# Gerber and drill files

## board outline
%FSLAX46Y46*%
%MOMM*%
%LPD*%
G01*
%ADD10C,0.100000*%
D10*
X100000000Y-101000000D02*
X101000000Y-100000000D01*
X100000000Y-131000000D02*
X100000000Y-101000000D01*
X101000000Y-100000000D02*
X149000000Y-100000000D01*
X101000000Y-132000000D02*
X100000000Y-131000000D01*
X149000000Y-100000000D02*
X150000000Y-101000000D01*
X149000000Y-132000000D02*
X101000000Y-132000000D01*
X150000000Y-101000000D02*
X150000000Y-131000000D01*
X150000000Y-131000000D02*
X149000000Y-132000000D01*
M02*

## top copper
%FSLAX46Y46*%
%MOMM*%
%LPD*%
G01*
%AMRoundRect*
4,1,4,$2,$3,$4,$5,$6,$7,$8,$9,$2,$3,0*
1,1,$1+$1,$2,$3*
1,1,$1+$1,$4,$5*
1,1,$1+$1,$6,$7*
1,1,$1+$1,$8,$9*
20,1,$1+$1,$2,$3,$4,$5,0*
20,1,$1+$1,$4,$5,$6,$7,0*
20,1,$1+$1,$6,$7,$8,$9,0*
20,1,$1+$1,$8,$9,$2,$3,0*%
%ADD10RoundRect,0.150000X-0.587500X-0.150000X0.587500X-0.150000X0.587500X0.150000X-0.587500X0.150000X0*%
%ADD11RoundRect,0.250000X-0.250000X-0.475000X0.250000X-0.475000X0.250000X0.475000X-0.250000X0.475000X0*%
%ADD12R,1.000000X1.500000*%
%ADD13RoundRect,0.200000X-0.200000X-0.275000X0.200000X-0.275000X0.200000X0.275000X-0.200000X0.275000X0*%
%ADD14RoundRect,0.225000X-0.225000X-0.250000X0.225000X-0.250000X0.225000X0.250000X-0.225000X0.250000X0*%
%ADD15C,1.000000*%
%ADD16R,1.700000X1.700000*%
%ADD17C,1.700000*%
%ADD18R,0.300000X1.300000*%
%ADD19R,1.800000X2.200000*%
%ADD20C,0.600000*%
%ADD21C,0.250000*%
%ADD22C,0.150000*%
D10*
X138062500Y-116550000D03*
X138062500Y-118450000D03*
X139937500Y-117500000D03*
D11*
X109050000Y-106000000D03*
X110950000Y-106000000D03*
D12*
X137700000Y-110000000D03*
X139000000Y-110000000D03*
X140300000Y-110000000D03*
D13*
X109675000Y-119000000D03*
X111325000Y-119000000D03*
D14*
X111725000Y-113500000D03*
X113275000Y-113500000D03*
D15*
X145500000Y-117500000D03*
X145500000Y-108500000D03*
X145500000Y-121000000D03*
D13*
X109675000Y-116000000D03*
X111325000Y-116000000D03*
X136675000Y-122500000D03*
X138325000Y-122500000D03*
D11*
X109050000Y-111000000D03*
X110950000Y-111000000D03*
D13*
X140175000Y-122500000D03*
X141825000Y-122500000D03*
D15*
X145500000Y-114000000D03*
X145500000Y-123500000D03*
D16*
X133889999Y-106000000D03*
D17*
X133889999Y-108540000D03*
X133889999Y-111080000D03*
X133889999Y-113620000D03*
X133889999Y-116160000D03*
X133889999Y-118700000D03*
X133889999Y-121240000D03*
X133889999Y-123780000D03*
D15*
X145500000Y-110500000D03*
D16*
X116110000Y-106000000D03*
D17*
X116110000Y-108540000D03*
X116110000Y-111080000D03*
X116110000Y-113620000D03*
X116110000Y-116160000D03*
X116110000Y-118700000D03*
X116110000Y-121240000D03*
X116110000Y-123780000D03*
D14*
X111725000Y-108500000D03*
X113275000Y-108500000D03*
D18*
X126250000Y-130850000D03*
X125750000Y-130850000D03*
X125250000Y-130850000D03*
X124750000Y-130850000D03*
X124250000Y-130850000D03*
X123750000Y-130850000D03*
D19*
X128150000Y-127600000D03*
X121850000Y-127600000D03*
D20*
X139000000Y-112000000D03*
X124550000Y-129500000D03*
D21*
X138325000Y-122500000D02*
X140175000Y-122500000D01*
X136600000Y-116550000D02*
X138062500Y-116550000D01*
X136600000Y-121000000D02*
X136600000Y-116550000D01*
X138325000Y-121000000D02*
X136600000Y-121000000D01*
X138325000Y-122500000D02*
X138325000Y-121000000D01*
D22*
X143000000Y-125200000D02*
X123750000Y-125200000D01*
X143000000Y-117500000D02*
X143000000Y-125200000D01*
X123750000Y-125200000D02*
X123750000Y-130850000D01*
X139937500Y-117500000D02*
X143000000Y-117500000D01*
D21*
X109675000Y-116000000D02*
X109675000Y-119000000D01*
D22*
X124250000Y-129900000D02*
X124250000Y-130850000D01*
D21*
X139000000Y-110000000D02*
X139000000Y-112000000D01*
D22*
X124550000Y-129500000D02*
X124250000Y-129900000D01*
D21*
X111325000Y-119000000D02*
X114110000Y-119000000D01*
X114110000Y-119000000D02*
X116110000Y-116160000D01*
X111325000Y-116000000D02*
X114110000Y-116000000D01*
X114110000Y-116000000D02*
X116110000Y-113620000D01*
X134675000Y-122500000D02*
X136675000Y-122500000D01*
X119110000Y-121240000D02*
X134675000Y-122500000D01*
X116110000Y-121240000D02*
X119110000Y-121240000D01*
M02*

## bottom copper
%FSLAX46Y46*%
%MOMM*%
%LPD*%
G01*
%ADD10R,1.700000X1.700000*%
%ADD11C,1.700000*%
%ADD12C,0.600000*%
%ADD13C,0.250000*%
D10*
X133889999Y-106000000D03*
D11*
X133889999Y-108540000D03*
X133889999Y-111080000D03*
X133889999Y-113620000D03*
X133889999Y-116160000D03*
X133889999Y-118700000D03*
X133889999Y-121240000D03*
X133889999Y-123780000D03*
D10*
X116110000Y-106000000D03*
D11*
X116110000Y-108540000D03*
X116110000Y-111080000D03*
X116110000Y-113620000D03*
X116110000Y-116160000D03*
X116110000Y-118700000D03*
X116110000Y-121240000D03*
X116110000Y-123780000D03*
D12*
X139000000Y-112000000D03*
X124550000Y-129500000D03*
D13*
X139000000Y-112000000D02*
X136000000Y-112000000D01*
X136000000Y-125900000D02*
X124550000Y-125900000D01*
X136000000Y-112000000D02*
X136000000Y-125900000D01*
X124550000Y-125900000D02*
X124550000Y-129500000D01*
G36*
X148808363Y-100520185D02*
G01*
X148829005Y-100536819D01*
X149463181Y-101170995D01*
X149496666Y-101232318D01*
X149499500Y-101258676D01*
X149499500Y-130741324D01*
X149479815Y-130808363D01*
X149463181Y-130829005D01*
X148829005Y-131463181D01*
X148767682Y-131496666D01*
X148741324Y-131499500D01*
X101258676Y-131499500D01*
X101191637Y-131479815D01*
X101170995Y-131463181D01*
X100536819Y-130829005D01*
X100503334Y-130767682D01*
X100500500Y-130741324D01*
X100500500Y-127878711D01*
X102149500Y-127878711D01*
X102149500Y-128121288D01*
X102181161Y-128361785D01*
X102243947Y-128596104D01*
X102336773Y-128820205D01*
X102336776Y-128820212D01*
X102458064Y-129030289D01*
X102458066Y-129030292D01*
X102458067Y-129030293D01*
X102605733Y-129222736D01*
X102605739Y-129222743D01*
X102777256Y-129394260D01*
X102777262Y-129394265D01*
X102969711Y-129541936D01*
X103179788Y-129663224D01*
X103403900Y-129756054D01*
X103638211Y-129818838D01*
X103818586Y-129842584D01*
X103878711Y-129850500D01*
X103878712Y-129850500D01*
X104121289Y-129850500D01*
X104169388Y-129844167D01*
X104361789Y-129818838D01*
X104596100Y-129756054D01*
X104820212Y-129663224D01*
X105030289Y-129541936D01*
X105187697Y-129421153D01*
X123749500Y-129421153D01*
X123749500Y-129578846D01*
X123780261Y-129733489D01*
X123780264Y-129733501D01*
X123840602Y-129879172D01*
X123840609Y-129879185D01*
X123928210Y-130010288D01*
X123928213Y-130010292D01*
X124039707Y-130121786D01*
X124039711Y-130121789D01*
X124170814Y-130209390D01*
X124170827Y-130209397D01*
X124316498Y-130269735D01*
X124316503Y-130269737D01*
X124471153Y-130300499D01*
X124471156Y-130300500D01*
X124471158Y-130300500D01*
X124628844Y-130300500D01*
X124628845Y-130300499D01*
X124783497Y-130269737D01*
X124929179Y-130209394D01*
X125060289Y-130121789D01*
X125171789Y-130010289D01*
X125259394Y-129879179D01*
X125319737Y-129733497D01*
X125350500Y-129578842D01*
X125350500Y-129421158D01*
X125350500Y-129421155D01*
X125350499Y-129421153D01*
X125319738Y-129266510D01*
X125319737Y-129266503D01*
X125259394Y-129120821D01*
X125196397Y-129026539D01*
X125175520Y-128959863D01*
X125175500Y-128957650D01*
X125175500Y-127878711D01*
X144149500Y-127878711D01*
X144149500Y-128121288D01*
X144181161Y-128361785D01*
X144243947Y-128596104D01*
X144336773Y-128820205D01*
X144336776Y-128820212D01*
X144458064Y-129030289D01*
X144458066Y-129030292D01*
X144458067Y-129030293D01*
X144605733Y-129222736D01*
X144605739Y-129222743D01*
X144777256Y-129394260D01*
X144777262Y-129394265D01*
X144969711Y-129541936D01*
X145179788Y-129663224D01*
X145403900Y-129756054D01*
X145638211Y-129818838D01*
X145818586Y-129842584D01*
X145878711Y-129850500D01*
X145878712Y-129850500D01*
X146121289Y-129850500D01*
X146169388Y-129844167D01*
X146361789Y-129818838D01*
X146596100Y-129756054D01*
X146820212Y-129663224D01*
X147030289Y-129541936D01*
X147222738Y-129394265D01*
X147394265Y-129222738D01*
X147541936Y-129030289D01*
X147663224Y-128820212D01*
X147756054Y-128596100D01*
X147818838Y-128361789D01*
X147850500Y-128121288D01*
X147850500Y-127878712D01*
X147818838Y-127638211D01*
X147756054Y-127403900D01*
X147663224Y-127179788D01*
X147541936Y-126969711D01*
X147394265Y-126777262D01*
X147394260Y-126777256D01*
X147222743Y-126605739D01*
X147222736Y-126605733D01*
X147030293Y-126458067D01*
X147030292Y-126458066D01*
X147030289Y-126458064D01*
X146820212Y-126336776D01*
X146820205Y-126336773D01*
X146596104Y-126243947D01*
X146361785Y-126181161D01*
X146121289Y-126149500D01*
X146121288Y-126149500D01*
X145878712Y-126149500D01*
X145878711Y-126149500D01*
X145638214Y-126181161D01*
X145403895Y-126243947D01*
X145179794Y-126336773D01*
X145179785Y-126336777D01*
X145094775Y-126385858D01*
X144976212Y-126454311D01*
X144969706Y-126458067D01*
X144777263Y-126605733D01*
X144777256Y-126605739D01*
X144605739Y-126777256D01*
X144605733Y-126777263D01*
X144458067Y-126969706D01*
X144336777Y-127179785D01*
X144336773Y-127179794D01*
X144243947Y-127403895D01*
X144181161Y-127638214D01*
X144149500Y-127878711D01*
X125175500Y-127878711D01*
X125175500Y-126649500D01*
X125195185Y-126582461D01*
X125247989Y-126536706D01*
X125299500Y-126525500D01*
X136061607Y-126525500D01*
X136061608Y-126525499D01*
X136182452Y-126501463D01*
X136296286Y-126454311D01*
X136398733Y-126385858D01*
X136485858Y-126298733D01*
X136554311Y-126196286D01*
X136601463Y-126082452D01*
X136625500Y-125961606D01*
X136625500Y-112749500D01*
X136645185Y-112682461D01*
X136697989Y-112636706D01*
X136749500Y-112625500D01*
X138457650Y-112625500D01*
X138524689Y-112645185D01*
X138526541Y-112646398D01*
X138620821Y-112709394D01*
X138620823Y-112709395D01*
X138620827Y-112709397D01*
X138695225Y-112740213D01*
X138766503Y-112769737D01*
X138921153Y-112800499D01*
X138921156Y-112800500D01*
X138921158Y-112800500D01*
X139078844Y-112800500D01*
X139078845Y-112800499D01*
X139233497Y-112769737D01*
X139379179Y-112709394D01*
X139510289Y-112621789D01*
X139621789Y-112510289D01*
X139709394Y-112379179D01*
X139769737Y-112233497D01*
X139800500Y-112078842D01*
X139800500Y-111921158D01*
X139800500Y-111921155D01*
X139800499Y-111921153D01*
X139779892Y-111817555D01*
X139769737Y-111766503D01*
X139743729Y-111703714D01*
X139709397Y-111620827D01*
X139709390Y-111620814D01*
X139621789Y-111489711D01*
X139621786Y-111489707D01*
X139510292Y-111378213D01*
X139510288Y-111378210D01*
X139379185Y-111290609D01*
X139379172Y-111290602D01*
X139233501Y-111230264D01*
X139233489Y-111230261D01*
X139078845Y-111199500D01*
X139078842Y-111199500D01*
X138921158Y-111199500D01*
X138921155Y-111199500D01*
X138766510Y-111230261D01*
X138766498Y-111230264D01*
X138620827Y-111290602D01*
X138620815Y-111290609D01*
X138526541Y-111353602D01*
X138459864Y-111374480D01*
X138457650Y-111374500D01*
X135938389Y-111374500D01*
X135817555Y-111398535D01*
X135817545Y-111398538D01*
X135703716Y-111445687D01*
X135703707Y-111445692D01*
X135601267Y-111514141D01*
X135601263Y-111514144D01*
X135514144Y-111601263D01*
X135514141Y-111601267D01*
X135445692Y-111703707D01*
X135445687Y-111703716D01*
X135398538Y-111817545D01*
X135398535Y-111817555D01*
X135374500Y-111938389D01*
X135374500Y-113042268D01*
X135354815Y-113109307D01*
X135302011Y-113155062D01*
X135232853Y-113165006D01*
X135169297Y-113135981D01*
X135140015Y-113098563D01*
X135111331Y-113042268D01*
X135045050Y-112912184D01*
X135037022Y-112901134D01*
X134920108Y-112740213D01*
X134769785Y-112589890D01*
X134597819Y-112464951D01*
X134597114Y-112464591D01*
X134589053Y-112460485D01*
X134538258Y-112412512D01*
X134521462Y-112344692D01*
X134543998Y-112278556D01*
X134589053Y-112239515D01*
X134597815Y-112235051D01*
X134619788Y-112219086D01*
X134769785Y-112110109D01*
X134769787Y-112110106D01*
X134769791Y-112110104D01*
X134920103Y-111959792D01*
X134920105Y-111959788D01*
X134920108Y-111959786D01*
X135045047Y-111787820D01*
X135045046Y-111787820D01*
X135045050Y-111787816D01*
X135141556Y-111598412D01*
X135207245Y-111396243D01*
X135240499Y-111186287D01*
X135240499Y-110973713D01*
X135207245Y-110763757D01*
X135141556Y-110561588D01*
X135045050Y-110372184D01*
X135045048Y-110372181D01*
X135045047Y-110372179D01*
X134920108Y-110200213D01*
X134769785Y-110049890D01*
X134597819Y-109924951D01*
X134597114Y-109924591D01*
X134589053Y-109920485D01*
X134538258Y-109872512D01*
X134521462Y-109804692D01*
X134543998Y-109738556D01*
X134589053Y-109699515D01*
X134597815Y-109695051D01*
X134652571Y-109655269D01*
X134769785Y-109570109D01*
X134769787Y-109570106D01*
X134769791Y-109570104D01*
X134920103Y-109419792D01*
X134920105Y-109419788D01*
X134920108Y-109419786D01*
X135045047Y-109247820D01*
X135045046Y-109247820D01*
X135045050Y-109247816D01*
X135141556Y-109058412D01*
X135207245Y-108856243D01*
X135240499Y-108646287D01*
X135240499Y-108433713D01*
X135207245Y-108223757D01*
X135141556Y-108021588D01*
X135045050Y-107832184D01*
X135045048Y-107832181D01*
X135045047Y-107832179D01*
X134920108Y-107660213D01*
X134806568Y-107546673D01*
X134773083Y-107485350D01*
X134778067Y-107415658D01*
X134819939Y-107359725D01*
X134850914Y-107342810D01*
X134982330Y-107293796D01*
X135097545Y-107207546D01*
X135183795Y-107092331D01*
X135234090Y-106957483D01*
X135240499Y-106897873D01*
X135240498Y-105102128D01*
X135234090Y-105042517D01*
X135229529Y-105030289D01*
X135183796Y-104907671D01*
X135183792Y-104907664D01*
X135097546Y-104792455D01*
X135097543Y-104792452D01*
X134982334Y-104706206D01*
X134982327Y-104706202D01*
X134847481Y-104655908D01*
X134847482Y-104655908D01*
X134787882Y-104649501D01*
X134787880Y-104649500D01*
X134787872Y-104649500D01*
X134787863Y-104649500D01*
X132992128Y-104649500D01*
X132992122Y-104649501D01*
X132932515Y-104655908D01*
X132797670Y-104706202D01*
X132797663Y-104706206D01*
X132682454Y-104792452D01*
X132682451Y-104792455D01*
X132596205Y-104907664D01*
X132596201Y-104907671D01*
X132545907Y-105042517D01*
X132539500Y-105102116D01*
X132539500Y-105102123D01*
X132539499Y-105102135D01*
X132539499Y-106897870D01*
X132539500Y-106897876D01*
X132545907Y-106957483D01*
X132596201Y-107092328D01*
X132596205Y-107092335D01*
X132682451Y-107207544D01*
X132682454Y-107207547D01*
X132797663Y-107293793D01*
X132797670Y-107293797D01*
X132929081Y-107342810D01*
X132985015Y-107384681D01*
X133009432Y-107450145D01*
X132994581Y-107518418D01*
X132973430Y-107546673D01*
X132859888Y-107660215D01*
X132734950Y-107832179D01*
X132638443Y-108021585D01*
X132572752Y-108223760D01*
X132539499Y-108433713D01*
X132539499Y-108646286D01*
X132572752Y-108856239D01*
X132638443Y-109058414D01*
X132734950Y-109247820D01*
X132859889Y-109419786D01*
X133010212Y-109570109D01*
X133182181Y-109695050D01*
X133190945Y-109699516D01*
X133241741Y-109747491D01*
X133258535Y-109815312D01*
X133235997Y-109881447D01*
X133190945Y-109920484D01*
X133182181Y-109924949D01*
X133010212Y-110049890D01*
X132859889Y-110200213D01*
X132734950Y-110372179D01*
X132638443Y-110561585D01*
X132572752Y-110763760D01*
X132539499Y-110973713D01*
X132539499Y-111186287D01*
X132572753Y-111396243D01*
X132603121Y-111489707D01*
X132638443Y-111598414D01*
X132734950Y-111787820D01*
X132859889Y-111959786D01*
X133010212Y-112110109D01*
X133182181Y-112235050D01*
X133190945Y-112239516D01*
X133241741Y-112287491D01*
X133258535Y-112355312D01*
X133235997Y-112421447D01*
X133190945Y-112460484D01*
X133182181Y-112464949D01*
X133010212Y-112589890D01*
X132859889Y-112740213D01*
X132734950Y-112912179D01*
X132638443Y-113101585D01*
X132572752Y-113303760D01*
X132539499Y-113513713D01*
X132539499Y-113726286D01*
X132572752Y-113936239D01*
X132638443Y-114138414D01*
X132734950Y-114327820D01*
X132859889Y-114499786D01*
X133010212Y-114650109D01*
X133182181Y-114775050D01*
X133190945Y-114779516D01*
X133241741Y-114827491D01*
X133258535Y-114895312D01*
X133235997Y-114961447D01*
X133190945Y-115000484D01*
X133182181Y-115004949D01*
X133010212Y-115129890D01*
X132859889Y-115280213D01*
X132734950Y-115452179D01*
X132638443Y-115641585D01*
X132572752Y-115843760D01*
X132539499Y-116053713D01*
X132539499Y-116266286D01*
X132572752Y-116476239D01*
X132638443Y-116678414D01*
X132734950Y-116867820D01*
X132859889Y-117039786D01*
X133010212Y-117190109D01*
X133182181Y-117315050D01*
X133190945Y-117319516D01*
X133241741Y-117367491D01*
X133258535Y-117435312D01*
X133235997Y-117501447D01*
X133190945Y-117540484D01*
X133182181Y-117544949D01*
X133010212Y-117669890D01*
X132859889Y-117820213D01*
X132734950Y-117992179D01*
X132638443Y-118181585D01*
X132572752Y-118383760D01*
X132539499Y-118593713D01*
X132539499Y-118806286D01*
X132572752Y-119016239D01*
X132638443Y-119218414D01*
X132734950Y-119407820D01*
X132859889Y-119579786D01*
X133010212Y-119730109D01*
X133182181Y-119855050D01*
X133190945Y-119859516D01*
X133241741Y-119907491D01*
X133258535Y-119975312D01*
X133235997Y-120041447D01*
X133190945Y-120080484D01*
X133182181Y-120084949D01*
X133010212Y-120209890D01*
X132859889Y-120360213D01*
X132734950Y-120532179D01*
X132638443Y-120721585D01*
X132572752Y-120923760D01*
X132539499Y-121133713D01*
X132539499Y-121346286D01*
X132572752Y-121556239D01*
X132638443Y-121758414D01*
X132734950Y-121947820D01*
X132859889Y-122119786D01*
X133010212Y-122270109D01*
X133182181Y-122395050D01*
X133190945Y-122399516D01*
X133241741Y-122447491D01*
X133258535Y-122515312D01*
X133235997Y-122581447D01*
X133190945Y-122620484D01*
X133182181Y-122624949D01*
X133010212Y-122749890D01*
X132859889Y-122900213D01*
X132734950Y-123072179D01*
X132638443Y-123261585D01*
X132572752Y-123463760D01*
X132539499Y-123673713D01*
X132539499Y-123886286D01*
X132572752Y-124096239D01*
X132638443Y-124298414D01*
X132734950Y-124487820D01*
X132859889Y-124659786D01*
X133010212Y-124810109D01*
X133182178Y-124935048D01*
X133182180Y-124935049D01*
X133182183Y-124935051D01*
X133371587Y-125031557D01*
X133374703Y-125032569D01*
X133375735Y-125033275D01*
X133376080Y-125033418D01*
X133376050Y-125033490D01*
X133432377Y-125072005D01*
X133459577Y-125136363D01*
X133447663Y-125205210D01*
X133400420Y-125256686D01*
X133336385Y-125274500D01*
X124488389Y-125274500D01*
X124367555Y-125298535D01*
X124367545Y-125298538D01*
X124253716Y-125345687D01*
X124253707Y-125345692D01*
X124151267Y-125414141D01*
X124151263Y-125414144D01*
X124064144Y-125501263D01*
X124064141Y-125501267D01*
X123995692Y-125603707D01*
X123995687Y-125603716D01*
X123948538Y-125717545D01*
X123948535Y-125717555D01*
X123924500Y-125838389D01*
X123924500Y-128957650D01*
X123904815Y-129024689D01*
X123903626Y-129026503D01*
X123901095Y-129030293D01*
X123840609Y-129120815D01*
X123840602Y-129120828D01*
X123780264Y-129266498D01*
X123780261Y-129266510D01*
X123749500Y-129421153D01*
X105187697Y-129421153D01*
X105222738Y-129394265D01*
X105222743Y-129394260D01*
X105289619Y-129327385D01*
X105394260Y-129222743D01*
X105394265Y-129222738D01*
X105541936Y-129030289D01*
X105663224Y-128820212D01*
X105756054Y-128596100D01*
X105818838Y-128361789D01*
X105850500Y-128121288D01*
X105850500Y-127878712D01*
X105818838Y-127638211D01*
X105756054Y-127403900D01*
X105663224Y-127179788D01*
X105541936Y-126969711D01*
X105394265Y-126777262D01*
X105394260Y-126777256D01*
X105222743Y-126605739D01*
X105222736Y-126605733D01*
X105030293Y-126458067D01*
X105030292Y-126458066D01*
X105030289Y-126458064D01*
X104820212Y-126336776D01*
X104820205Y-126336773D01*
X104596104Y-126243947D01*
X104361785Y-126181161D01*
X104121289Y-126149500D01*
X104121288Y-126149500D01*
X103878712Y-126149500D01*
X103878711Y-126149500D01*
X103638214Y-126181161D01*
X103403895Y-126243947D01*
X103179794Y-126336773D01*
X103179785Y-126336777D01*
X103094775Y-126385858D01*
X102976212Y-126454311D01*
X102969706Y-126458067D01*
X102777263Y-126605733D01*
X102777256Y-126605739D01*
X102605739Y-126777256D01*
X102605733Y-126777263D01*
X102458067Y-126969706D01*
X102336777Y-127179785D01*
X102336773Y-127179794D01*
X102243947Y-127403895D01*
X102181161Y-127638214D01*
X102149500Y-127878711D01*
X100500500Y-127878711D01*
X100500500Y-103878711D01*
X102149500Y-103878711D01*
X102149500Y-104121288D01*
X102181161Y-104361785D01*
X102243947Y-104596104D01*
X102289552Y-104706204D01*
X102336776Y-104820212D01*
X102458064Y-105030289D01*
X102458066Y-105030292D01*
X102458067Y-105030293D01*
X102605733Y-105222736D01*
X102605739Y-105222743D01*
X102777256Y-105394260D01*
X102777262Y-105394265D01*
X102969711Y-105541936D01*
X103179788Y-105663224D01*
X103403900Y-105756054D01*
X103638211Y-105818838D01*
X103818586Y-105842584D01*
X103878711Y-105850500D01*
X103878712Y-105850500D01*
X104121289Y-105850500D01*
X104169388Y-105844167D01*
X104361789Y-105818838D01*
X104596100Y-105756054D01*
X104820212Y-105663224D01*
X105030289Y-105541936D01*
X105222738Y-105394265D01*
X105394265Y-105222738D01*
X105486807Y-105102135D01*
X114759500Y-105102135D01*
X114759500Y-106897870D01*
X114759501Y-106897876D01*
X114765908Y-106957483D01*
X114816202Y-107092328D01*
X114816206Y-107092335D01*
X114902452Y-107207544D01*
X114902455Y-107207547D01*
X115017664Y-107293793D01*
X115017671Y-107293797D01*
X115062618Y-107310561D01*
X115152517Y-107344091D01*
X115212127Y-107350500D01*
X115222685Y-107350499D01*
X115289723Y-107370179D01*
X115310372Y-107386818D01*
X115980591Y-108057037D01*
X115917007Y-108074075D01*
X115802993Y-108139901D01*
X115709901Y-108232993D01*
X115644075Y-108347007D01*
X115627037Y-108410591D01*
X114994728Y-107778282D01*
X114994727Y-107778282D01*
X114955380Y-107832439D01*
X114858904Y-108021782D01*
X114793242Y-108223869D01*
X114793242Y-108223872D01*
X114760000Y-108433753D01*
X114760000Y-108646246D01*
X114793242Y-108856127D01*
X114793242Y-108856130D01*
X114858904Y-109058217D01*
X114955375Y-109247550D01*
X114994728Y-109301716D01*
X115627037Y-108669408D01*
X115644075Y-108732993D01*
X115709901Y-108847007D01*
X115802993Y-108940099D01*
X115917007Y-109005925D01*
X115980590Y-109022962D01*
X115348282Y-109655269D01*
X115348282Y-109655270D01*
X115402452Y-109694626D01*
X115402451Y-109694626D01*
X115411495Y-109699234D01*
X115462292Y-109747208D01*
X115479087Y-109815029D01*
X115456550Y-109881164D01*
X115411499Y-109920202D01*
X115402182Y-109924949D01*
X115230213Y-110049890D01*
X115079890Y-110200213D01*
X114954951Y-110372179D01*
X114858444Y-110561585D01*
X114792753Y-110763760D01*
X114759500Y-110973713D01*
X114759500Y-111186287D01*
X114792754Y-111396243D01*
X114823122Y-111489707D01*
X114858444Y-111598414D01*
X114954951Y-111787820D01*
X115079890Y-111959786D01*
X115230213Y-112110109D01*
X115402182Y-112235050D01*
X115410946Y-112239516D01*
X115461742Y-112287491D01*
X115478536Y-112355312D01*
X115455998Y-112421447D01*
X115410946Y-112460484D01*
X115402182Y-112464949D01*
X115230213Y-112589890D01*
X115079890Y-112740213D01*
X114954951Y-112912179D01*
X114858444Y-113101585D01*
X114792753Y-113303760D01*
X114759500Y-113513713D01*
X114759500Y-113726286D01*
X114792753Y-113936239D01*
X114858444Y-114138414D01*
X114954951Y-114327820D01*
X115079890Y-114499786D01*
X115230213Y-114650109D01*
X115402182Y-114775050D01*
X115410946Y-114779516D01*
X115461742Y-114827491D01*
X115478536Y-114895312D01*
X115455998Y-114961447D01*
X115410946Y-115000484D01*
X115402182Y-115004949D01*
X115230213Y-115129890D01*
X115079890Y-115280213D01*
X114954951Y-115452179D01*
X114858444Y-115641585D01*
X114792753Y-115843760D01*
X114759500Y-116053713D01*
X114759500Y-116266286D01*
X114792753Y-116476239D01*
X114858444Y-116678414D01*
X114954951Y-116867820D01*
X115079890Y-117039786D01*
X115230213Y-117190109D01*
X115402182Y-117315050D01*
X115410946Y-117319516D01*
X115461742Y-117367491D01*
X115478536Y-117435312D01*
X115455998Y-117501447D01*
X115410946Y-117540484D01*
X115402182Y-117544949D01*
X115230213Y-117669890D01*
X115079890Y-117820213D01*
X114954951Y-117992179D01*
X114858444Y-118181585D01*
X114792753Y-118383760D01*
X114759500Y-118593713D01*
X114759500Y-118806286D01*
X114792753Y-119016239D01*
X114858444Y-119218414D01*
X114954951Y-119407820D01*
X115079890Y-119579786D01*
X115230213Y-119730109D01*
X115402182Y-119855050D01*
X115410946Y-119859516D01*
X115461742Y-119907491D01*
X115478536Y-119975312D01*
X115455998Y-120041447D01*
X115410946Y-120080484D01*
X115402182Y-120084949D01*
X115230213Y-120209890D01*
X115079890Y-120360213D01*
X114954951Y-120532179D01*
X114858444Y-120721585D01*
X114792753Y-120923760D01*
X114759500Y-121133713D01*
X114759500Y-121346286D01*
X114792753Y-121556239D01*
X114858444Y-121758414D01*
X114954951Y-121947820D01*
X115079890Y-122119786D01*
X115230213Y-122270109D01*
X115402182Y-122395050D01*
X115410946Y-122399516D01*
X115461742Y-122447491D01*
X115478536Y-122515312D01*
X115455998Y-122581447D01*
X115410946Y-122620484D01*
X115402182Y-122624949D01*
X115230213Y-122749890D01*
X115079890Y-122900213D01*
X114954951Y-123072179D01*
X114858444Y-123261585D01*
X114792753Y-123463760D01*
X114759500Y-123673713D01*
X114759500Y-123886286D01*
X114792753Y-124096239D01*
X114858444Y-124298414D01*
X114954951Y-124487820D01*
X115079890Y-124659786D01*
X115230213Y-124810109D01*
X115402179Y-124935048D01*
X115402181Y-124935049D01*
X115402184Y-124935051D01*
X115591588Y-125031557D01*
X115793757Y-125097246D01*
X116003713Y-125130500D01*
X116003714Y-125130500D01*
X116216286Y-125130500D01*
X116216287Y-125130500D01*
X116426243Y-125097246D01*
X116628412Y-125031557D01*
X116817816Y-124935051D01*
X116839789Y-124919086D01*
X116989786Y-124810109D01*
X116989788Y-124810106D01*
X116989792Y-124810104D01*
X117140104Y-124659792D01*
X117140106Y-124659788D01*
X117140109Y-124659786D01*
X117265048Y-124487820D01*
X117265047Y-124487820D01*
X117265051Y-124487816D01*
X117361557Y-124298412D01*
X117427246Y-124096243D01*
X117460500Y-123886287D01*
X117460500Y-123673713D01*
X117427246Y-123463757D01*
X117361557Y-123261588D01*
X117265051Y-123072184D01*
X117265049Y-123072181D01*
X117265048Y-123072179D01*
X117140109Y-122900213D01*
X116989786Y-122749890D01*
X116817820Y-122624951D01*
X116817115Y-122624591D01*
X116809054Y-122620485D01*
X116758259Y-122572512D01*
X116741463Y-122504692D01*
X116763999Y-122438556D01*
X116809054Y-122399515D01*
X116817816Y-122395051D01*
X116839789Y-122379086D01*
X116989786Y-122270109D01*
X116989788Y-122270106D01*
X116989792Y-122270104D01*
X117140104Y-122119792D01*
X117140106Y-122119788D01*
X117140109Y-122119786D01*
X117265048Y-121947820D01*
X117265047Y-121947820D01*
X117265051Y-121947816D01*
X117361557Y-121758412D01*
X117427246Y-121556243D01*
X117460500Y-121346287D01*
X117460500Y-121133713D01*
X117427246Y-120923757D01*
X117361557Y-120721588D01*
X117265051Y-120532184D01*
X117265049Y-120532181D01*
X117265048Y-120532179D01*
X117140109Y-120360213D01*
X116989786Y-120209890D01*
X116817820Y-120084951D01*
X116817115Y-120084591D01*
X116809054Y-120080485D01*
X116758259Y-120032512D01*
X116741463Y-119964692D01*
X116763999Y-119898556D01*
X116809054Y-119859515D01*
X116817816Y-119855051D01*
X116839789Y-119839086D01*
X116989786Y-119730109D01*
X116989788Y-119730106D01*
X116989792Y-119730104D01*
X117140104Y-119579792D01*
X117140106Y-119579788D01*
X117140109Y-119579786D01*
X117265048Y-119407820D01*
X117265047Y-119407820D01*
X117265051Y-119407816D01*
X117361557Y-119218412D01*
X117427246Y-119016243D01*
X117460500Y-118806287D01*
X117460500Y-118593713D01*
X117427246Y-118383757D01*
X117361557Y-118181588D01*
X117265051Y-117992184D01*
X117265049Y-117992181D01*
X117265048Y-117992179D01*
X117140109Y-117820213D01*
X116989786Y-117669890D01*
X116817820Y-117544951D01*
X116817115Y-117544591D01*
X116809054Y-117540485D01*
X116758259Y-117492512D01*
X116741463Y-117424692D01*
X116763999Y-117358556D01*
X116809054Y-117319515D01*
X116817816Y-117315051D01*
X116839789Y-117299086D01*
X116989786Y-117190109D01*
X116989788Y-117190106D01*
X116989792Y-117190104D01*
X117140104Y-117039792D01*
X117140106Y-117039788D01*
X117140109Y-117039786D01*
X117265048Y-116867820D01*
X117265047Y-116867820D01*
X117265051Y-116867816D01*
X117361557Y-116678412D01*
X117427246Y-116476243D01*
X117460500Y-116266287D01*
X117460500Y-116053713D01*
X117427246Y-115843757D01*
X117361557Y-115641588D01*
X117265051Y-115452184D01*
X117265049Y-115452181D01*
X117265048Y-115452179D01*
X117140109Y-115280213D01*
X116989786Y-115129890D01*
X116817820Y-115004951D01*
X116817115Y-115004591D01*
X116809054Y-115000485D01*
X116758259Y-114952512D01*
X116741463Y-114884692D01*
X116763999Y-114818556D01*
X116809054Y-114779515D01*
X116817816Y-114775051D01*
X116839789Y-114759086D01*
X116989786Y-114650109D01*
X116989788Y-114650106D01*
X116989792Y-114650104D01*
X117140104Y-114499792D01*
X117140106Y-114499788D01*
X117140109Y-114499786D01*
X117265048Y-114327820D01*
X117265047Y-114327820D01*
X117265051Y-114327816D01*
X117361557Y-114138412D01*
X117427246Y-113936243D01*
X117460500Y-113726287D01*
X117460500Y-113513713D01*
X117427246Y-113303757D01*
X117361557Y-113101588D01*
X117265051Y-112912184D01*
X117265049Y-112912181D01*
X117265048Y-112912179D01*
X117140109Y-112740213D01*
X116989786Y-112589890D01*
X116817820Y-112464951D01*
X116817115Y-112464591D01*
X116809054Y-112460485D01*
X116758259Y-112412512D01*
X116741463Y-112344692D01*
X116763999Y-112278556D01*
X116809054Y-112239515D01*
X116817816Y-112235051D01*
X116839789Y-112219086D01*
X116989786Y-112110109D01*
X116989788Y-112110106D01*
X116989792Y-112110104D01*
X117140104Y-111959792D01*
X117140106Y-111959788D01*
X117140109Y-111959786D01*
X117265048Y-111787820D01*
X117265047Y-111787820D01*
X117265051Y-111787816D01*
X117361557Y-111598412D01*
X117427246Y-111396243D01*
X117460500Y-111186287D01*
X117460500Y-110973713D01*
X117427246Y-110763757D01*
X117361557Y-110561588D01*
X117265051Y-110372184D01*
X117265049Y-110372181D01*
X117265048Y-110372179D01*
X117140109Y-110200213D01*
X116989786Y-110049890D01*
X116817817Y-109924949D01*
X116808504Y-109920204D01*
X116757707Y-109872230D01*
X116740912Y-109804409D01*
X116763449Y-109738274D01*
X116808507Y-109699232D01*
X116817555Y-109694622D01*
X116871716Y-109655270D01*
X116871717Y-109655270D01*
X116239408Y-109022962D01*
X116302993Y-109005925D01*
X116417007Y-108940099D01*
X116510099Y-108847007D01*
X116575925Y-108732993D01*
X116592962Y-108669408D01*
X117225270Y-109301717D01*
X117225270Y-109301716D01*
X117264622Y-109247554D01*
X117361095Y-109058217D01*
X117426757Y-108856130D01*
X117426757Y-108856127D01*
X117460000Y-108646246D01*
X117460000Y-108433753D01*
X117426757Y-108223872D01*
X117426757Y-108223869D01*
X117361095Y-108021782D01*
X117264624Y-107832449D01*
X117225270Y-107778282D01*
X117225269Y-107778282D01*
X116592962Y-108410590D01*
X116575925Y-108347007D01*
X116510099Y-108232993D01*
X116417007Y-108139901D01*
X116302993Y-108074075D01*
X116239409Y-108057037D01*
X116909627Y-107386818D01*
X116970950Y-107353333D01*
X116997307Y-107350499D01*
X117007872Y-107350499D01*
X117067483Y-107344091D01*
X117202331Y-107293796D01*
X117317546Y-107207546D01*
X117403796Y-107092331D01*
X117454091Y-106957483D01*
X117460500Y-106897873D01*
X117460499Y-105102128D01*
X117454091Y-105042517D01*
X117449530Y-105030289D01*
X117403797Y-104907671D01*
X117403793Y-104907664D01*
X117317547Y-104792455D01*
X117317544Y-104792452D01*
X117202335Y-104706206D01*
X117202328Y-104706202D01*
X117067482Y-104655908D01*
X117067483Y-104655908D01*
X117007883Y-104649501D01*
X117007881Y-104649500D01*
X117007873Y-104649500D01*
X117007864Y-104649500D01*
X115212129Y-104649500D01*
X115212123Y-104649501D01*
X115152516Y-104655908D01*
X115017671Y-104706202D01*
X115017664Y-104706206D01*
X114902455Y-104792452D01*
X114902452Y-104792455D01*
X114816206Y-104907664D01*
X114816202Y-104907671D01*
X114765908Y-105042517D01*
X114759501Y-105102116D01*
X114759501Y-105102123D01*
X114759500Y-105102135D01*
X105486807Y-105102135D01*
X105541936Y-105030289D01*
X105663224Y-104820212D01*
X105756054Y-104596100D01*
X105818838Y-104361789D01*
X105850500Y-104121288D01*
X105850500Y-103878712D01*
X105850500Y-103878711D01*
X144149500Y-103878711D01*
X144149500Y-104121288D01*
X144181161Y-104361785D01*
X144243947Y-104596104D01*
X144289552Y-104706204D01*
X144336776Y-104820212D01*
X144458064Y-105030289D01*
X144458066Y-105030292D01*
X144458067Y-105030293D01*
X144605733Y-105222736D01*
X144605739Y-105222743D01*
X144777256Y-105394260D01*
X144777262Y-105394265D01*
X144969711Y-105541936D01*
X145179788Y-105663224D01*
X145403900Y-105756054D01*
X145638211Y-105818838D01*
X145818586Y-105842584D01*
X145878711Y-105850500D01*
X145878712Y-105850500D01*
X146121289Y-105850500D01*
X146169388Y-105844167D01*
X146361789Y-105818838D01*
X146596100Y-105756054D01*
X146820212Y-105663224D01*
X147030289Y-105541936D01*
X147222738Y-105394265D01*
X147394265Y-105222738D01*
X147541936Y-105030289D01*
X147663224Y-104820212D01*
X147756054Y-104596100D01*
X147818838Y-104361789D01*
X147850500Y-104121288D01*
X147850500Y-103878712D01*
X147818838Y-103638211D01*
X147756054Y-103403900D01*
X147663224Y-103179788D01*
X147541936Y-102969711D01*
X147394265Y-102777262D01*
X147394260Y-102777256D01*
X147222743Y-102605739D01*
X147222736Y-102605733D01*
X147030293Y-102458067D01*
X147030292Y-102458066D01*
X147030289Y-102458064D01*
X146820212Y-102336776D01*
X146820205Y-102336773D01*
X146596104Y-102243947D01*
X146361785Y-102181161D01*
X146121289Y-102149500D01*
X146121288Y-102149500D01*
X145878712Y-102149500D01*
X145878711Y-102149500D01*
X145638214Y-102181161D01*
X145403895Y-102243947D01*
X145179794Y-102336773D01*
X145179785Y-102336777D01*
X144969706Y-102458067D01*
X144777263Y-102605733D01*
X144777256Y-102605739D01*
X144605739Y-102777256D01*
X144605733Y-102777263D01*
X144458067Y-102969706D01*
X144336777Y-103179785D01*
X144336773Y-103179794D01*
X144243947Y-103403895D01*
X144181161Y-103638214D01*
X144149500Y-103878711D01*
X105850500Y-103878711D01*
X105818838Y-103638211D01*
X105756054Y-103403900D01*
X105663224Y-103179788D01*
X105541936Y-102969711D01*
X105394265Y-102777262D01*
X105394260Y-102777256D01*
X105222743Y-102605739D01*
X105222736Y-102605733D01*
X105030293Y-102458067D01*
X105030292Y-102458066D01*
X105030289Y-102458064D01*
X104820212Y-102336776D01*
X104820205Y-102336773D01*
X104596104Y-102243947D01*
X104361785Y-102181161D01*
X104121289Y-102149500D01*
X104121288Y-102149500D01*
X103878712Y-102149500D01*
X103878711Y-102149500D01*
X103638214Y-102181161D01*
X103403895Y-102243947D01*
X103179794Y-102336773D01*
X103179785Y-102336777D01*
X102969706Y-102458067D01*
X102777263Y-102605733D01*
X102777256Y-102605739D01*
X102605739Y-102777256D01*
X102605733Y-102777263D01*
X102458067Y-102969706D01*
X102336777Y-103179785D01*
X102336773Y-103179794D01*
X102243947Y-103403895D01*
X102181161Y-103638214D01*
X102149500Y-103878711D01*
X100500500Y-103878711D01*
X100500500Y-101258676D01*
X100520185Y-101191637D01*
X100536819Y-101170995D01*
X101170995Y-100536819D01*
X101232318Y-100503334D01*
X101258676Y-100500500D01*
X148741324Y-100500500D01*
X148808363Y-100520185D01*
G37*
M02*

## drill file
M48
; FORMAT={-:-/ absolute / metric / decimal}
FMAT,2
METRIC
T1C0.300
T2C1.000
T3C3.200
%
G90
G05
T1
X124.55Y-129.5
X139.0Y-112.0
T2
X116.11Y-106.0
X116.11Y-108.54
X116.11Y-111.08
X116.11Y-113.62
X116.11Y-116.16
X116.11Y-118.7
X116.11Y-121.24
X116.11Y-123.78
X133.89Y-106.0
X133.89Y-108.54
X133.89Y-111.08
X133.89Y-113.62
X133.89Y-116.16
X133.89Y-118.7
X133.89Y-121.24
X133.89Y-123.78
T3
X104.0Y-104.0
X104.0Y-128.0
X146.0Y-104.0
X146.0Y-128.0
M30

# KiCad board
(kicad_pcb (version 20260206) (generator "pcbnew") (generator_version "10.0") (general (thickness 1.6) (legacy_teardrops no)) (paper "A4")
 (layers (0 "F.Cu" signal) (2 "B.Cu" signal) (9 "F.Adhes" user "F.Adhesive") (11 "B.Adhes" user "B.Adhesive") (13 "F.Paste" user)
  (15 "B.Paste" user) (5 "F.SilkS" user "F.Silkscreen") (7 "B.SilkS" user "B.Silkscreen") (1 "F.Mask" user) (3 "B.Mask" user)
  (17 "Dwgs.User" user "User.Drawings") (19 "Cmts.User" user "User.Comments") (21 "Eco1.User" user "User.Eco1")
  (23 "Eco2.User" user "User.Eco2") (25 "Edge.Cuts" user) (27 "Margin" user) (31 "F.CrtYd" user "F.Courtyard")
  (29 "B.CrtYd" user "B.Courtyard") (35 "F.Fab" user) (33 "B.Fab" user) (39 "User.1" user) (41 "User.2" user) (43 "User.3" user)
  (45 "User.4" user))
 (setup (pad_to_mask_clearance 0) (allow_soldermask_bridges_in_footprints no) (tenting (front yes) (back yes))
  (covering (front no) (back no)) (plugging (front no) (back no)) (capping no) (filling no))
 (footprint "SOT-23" (layer "F.Cu") (at 139 117.5)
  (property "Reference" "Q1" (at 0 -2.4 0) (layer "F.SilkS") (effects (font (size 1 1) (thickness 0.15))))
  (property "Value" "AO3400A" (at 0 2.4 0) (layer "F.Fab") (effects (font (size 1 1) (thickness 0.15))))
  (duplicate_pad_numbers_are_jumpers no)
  (pad "1" smd roundrect (at -0.9375 -0.95) (size 1.475 0.6) (layers "F.Cu" "F.Mask" "F.Paste") (roundrect_rratio 0.25) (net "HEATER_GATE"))
  (pad "2" smd roundrect (at -0.9375 0.95) (size 1.475 0.6) (layers "F.Cu" "F.Mask" "F.Paste") (roundrect_rratio 0.25) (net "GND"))
  (pad "3" smd roundrect (at 0.9375 0) (size 1.475 0.6) (layers "F.Cu" "F.Mask" "F.Paste") (roundrect_rratio 0.25) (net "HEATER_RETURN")))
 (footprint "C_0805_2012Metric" (layer "F.Cu") (at 110 106)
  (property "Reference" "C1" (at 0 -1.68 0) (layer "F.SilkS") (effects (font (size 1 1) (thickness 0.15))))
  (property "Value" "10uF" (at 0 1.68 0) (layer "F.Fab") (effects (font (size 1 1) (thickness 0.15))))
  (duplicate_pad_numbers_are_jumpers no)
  (pad "1" smd roundrect (at -0.95 0) (size 1 1.45) (layers "F.Cu" "F.Mask" "F.Paste") (roundrect_rratio 0.25) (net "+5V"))
  (pad "2" smd roundrect (at 0.95 0) (size 1 1.45) (layers "F.Cu" "F.Mask" "F.Paste") (roundrect_rratio 0.25) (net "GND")))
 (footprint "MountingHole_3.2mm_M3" (layer "F.Cu") (at 104 128)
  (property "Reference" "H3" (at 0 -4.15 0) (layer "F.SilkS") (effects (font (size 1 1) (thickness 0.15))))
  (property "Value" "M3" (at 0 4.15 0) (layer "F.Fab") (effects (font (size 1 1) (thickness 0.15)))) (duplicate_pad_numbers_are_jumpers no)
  (pad "" np_thru_hole circle (at 0 0) (size 3.2 3.2) (drill 3.2) (layers "*.Cu" "*.Mask")))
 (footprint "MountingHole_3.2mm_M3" (layer "F.Cu") (at 146 128)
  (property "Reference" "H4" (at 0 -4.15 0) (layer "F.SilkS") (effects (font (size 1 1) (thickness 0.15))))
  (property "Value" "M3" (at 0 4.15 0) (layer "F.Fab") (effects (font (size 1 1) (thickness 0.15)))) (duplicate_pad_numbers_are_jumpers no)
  (pad "" np_thru_hole circle (at 0 0) (size 3.2 3.2) (drill 3.2) (layers "*.Cu" "*.Mask")))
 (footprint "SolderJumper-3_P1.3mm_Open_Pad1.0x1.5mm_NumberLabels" (layer "F.Cu") (at 139 110)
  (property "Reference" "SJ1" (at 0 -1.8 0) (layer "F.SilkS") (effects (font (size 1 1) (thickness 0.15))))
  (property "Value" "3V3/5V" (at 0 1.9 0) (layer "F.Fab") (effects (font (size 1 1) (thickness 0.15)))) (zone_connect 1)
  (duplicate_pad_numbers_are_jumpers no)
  (pad "1" smd rect (at -1.3 0) (size 1 1.5) (layers "F.Cu" "F.Mask") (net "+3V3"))
  (pad "2" smd rect (at 0 0) (size 1 1.5) (layers "F.Cu" "F.Mask") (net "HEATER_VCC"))
  (pad "3" smd rect (at 1.3 0) (size 1 1.5) (layers "F.Cu" "F.Mask") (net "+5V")))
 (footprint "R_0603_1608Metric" (layer "F.Cu") (at 110.5 119)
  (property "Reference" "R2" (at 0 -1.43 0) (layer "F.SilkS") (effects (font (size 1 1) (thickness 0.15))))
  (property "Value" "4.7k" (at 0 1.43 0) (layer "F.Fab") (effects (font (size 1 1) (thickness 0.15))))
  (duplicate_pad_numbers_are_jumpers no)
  (pad "1" smd roundrect (at -0.825 0) (size 0.8 0.95) (layers "F.Cu" "F.Mask" "F.Paste") (roundrect_rratio 0.25) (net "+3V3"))
  (pad "2" smd roundrect (at 0.825 0) (size 0.8 0.95) (layers "F.Cu" "F.Mask" "F.Paste") (roundrect_rratio 0.25) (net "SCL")))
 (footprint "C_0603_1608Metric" (layer "F.Cu") (at 112.5 113.5)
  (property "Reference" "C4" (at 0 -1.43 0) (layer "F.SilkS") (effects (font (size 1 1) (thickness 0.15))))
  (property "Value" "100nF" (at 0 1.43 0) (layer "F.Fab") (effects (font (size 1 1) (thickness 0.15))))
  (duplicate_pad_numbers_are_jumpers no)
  (pad "1" smd roundrect (at -0.775 0) (size 0.9 0.95) (layers "F.Cu" "F.Mask" "F.Paste") (roundrect_rratio 0.25) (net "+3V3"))
  (pad "2" smd roundrect (at 0.775 0) (size 0.9 0.95) (layers "F.Cu" "F.Mask" "F.Paste") (roundrect_rratio 0.25) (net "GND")))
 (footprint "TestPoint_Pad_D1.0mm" (layer "F.Cu") (at 145.5 117.5)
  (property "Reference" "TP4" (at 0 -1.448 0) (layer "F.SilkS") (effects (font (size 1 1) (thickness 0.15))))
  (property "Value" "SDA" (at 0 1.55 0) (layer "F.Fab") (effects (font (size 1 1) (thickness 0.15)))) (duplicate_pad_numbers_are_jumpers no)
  (pad "1" smd circle (at 0 0) (size 1 1) (layers "F.Cu" "F.Mask") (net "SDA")))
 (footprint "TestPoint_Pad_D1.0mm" (layer "F.Cu") (at 145.5 108.5)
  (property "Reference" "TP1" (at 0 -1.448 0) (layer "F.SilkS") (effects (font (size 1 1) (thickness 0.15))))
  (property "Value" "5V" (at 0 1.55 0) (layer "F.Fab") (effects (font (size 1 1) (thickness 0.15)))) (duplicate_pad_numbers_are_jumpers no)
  (pad "1" smd circle (at 0 0) (size 1 1) (layers "F.Cu" "F.Mask") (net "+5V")))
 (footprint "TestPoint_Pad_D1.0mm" (layer "F.Cu") (at 145.5 121)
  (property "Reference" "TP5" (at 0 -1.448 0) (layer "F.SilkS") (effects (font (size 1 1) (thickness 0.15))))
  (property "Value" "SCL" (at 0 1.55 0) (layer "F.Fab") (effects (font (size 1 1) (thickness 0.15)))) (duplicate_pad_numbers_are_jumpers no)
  (pad "1" smd circle (at 0 0) (size 1 1) (layers "F.Cu" "F.Mask") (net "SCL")))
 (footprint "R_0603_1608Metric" (layer "F.Cu") (at 110.5 116)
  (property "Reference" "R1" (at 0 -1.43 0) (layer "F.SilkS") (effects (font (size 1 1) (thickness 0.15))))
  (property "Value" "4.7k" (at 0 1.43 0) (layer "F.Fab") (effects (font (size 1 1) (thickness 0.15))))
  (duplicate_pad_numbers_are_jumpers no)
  (pad "1" smd roundrect (at -0.825 0) (size 0.8 0.95) (layers "F.Cu" "F.Mask" "F.Paste") (roundrect_rratio 0.25) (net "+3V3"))
  (pad "2" smd roundrect (at 0.825 0) (size 0.8 0.95) (layers "F.Cu" "F.Mask" "F.Paste") (roundrect_rratio 0.25) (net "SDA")))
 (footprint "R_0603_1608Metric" (layer "F.Cu") (at 137.5 122.5)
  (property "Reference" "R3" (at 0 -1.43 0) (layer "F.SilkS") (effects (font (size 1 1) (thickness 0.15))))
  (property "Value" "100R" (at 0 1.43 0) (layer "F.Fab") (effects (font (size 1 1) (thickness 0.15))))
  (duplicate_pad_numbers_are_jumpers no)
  (pad "1" smd roundrect (at -0.825 0) (size 0.8 0.95) (layers "F.Cu" "F.Mask" "F.Paste") (roundrect_rratio 0.25) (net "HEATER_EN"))
  (pad "2" smd roundrect (at 0.825 0) (size 0.8 0.95) (layers "F.Cu" "F.Mask" "F.Paste") (roundrect_rratio 0.25) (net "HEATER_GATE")))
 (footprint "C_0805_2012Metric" (layer "F.Cu") (at 110 111)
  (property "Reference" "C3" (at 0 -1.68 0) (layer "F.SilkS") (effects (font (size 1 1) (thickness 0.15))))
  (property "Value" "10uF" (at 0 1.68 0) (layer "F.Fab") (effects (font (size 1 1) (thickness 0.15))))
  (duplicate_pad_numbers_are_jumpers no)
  (pad "1" smd roundrect (at -0.95 0) (size 1 1.45) (layers "F.Cu" "F.Mask" "F.Paste") (roundrect_rratio 0.25) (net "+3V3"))
  (pad "2" smd roundrect (at 0.95 0) (size 1 1.45) (layers "F.Cu" "F.Mask" "F.Paste") (roundrect_rratio 0.25) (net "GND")))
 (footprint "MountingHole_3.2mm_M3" (layer "F.Cu") (at 104 104)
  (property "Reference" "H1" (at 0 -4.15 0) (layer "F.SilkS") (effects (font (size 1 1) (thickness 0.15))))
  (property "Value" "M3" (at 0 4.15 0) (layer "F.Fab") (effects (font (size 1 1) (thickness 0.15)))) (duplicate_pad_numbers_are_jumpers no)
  (pad "" np_thru_hole circle (at 0 0) (size 3.2 3.2) (drill 3.2) (layers "*.Cu" "*.Mask")))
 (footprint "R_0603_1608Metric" (layer "F.Cu") (at 141 122.5)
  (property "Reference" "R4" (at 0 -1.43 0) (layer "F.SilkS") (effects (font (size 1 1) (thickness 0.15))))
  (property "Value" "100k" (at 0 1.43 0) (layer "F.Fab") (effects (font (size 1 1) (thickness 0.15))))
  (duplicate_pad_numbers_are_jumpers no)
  (pad "1" smd roundrect (at -0.825 0) (size 0.8 0.95) (layers "F.Cu" "F.Mask" "F.Paste") (roundrect_rratio 0.25) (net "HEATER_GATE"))
  (pad "2" smd roundrect (at 0.825 0) (size 0.8 0.95) (layers "F.Cu" "F.Mask" "F.Paste") (roundrect_rratio 0.25) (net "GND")))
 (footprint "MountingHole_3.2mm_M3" (layer "F.Cu") (at 146 104)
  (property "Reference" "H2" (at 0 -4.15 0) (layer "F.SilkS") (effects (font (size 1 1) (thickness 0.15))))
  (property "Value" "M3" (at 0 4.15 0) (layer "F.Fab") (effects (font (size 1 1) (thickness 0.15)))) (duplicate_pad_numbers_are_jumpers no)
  (pad "" np_thru_hole circle (at 0 0) (size 3.2 3.2) (drill 3.2) (layers "*.Cu" "*.Mask")))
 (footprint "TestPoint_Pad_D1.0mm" (layer "F.Cu") (at 145.5 114)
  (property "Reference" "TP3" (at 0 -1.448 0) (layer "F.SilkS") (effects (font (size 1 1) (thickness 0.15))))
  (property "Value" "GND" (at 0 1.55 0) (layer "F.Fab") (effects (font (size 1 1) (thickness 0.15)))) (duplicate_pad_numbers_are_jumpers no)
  (pad "1" smd circle (at 0 0) (size 1 1) (layers "F.Cu" "F.Mask") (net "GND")))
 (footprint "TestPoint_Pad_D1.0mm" (layer "F.Cu") (at 145.5 123.5)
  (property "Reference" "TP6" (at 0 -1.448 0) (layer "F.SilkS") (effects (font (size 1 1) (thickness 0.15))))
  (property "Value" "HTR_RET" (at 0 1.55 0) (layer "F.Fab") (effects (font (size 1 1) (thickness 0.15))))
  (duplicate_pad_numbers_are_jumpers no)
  (pad "1" smd circle (at 0 0) (size 1 1) (layers "F.Cu" "F.Mask") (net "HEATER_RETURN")))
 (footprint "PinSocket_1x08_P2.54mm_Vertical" (layer "F.Cu") (at 133.889999 106)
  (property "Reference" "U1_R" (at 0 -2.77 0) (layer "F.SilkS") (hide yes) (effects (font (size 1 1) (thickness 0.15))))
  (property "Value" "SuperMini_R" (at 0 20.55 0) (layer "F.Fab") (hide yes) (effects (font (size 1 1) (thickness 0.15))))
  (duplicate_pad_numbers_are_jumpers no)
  (pad "1" thru_hole rect (at 0 0) (size 1.7 1.7) (drill 1) (layers "*.Cu" "*.Mask") (remove_unused_layers no))
  (pad "2" thru_hole circle (at 0 2.54) (size 1.7 1.7) (drill 1) (layers "*.Cu" "*.Mask") (remove_unused_layers no))
  (pad "3" thru_hole circle (at 0 5.08) (size 1.7 1.7) (drill 1) (layers "*.Cu" "*.Mask") (remove_unused_layers no))
  (pad "4" thru_hole circle (at 0 7.62) (size 1.7 1.7) (drill 1) (layers "*.Cu" "*.Mask") (remove_unused_layers no))
  (pad "5" thru_hole circle (at 0 10.16) (size 1.7 1.7) (drill 1) (layers "*.Cu" "*.Mask") (remove_unused_layers no))
  (pad "6" thru_hole circle (at 0 12.7) (size 1.7 1.7) (drill 1) (layers "*.Cu" "*.Mask") (remove_unused_layers no) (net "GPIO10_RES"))
  (pad "7" thru_hole circle (at 0 15.24) (size 1.7 1.7) (drill 1) (layers "*.Cu" "*.Mask") (remove_unused_layers no))
  (pad "8" thru_hole circle (at 0 17.78) (size 1.7 1.7) (drill 1) (layers "*.Cu" "*.Mask") (remove_unused_layers no)))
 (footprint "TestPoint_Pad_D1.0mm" (layer "F.Cu") (at 145.5 110.5)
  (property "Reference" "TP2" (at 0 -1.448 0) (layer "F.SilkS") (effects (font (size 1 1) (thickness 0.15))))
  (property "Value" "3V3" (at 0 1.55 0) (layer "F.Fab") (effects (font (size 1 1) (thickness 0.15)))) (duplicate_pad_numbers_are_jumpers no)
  (pad "1" smd circle (at 0 0) (size 1 1) (layers "F.Cu" "F.Mask") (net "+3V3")))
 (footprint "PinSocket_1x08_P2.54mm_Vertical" (layer "F.Cu") (at 116.11 106)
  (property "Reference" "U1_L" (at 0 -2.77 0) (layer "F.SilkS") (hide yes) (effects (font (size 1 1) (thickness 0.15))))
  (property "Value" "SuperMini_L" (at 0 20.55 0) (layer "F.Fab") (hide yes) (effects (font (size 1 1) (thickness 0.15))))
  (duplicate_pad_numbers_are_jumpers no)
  (pad "1" thru_hole rect (at 0 0) (size 1.7 1.7) (drill 1) (layers "*.Cu" "*.Mask") (remove_unused_layers no) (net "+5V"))
  (pad "2" thru_hole circle (at 0 2.54) (size 1.7 1.7) (drill 1) (layers "*.Cu" "*.Mask") (remove_unused_layers no) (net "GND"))
  (pad "3" thru_hole circle (at 0 5.08) (size 1.7 1.7) (drill 1) (layers "*.Cu" "*.Mask") (remove_unused_layers no) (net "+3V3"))
  (pad "4" thru_hole circle (at 0 7.62) (size 1.7 1.7) (drill 1) (layers "*.Cu" "*.Mask") (remove_unused_layers no) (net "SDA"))
  (pad "5" thru_hole circle (at 0 10.16) (size 1.7 1.7) (drill 1) (layers "*.Cu" "*.Mask") (remove_unused_layers no) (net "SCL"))
  (pad "6" thru_hole circle (at 0 12.7) (size 1.7 1.7) (drill 1) (layers "*.Cu" "*.Mask") (remove_unused_layers no))
  (pad "7" thru_hole circle (at 0 15.24) (size 1.7 1.7) (drill 1) (layers "*.Cu" "*.Mask") (remove_unused_layers no) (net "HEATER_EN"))
  (pad "8" thru_hole circle (at 0 17.78) (size 1.7 1.7) (drill 1) (layers "*.Cu" "*.Mask") (remove_unused_layers no)))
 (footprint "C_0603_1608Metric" (layer "F.Cu") (at 112.5 108.5)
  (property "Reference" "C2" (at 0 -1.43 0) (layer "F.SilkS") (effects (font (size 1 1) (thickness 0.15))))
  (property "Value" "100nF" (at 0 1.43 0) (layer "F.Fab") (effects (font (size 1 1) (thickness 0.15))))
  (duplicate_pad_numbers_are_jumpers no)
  (pad "1" smd roundrect (at -0.775 0) (size 0.9 0.95) (layers "F.Cu" "F.Mask" "F.Paste") (roundrect_rratio 0.25) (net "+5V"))
  (pad "2" smd roundrect (at 0.775 0) (size 0.9 0.95) (layers "F.Cu" "F.Mask" "F.Paste") (roundrect_rratio 0.25) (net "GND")))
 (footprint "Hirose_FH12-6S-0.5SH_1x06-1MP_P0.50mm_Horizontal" (layer "F.Cu") (at 125 129 180)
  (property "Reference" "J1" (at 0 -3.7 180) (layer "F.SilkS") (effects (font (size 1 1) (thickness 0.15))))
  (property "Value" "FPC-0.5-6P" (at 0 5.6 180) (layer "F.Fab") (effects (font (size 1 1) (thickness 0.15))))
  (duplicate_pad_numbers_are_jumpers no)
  (pad "1" smd rect (at -1.25 -1.85 180) (size 0.3 1.3) (layers "F.Cu" "F.Mask" "F.Paste") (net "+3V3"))
  (pad "2" smd rect (at -0.75 -1.85 180) (size 0.3 1.3) (layers "F.Cu" "F.Mask" "F.Paste") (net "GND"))
  (pad "3" smd rect (at -0.25 -1.85 180) (size 0.3 1.3) (layers "F.Cu" "F.Mask" "F.Paste") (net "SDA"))
  (pad "4" smd rect (at 0.25 -1.85 180) (size 0.3 1.3) (layers "F.Cu" "F.Mask" "F.Paste") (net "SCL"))
  (pad "5" smd rect (at 0.75 -1.85 180) (size 0.3 1.3) (layers "F.Cu" "F.Mask" "F.Paste") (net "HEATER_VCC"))
  (pad "6" smd rect (at 1.25 -1.85 180) (size 0.3 1.3) (layers "F.Cu" "F.Mask" "F.Paste") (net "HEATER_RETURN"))
  (pad "MP" smd rect (at -3.15 1.4 180) (size 1.8 2.2) (layers "F.Cu" "F.Mask" "F.Paste") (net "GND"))
  (pad "MP" smd rect (at 3.15 1.4 180) (size 1.8 2.2) (layers "F.Cu" "F.Mask" "F.Paste") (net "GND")))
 (gr_line (start 100 101) (end 101 100) (stroke (width 0.1) (type default)) (layer "Edge.Cuts"))
 (gr_line (start 100 131) (end 100 101) (stroke (width 0.1) (type default)) (layer "Edge.Cuts"))
 (gr_line (start 101 100) (end 149 100) (stroke (width 0.1) (type default)) (layer "Edge.Cuts"))
 (gr_line (start 101 132) (end 100 131) (stroke (width 0.1) (type default)) (layer "Edge.Cuts"))
 (gr_line (start 149 100) (end 150 101) (stroke (width 0.1) (type default)) (layer "Edge.Cuts"))
 (gr_line (start 149 132) (end 101 132) (stroke (width 0.1) (type default)) (layer "Edge.Cuts"))
 (gr_line (start 150 101) (end 150 131) (stroke (width 0.1) (type default)) (layer "Edge.Cuts"))
 (gr_line (start 150 131) (end 149 132) (stroke (width 0.1) (type default)) (layer "Edge.Cuts"))
 (segment (start 138.325 122.5) (end 140.175 122.5) (width 0.25) (layer "F.Cu") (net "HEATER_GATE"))
 (segment (start 136.6 116.55) (end 138.0625 116.55) (width 0.25) (layer "F.Cu") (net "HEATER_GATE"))
 (segment (start 136.6 121) (end 136.6 116.55) (width 0.25) (layer "F.Cu") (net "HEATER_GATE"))
 (segment (start 138.325 121) (end 136.6 121) (width 0.25) (layer "F.Cu") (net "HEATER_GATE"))
 (segment (start 138.325 122.5) (end 138.325 121) (width 0.25) (layer "F.Cu") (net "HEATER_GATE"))
 (segment (start 143 125.2) (end 123.75 125.2) (width 0.15) (layer "F.Cu") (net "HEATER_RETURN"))
 (segment (start 143 117.5) (end 143 125.2) (width 0.15) (layer "F.Cu") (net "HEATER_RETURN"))
 (segment (start 123.75 125.2) (end 123.75 130.85) (width 0.15) (layer "F.Cu") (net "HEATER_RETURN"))
 (segment (start 139.9375 117.5) (end 143 117.5) (width 0.15) (layer "F.Cu") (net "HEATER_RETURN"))
 (segment (start 109.675 116) (end 109.675 119) (width 0.25) (layer "F.Cu") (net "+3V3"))
 (segment (start 124.25 129.9) (end 124.25 130.85) (width 0.15) (layer "F.Cu") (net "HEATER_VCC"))
 (segment (start 139 110) (end 139 112) (width 0.25) (layer "F.Cu") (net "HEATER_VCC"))
 (segment (start 124.55 129.5) (end 124.25 129.9) (width 0.15) (layer "F.Cu") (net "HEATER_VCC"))
 (via (at 139 112) (size 0.6) (drill 0.3) (layers "F.Cu" "B.Cu") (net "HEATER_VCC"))
 (via (at 124.55 129.5) (size 0.6) (drill 0.3) (layers "F.Cu" "B.Cu") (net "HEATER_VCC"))
 (segment (start 139 112) (end 136 112) (width 0.25) (layer "B.Cu") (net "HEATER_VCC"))
 (segment (start 136 125.9) (end 124.55 125.9) (width 0.25) (layer "B.Cu") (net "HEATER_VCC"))
 (segment (start 136 112) (end 136 125.9) (width 0.25) (layer "B.Cu") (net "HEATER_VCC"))
 (segment (start 124.55 125.9) (end 124.55 129.5) (width 0.25) (layer "B.Cu") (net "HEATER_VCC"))
 (segment (start 111.325 119) (end 114.11 119) (width 0.25) (layer "F.Cu") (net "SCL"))
 (segment (start 114.11 119) (end 116.11 116.16) (width 0.25) (layer "F.Cu") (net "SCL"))
 (segment (start 111.325 116) (end 114.11 116) (width 0.25) (layer "F.Cu") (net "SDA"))
 (segment (start 114.11 116) (end 116.11 113.62) (width 0.25) (layer "F.Cu") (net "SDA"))
 (segment (start 134.675 122.5) (end 136.675 122.5) (width 0.25) (layer "F.Cu") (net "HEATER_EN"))
 (segment (start 119.11 121.24) (end 134.675 122.5) (width 0.25) (layer "F.Cu") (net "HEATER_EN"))
 (segment (start 116.11 121.24) (end 119.11 121.24) (width 0.25) (layer "F.Cu") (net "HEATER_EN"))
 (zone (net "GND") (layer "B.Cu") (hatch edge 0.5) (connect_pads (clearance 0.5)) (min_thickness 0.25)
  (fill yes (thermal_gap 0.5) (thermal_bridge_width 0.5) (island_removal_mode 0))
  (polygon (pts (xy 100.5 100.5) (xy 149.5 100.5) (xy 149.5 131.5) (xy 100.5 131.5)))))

